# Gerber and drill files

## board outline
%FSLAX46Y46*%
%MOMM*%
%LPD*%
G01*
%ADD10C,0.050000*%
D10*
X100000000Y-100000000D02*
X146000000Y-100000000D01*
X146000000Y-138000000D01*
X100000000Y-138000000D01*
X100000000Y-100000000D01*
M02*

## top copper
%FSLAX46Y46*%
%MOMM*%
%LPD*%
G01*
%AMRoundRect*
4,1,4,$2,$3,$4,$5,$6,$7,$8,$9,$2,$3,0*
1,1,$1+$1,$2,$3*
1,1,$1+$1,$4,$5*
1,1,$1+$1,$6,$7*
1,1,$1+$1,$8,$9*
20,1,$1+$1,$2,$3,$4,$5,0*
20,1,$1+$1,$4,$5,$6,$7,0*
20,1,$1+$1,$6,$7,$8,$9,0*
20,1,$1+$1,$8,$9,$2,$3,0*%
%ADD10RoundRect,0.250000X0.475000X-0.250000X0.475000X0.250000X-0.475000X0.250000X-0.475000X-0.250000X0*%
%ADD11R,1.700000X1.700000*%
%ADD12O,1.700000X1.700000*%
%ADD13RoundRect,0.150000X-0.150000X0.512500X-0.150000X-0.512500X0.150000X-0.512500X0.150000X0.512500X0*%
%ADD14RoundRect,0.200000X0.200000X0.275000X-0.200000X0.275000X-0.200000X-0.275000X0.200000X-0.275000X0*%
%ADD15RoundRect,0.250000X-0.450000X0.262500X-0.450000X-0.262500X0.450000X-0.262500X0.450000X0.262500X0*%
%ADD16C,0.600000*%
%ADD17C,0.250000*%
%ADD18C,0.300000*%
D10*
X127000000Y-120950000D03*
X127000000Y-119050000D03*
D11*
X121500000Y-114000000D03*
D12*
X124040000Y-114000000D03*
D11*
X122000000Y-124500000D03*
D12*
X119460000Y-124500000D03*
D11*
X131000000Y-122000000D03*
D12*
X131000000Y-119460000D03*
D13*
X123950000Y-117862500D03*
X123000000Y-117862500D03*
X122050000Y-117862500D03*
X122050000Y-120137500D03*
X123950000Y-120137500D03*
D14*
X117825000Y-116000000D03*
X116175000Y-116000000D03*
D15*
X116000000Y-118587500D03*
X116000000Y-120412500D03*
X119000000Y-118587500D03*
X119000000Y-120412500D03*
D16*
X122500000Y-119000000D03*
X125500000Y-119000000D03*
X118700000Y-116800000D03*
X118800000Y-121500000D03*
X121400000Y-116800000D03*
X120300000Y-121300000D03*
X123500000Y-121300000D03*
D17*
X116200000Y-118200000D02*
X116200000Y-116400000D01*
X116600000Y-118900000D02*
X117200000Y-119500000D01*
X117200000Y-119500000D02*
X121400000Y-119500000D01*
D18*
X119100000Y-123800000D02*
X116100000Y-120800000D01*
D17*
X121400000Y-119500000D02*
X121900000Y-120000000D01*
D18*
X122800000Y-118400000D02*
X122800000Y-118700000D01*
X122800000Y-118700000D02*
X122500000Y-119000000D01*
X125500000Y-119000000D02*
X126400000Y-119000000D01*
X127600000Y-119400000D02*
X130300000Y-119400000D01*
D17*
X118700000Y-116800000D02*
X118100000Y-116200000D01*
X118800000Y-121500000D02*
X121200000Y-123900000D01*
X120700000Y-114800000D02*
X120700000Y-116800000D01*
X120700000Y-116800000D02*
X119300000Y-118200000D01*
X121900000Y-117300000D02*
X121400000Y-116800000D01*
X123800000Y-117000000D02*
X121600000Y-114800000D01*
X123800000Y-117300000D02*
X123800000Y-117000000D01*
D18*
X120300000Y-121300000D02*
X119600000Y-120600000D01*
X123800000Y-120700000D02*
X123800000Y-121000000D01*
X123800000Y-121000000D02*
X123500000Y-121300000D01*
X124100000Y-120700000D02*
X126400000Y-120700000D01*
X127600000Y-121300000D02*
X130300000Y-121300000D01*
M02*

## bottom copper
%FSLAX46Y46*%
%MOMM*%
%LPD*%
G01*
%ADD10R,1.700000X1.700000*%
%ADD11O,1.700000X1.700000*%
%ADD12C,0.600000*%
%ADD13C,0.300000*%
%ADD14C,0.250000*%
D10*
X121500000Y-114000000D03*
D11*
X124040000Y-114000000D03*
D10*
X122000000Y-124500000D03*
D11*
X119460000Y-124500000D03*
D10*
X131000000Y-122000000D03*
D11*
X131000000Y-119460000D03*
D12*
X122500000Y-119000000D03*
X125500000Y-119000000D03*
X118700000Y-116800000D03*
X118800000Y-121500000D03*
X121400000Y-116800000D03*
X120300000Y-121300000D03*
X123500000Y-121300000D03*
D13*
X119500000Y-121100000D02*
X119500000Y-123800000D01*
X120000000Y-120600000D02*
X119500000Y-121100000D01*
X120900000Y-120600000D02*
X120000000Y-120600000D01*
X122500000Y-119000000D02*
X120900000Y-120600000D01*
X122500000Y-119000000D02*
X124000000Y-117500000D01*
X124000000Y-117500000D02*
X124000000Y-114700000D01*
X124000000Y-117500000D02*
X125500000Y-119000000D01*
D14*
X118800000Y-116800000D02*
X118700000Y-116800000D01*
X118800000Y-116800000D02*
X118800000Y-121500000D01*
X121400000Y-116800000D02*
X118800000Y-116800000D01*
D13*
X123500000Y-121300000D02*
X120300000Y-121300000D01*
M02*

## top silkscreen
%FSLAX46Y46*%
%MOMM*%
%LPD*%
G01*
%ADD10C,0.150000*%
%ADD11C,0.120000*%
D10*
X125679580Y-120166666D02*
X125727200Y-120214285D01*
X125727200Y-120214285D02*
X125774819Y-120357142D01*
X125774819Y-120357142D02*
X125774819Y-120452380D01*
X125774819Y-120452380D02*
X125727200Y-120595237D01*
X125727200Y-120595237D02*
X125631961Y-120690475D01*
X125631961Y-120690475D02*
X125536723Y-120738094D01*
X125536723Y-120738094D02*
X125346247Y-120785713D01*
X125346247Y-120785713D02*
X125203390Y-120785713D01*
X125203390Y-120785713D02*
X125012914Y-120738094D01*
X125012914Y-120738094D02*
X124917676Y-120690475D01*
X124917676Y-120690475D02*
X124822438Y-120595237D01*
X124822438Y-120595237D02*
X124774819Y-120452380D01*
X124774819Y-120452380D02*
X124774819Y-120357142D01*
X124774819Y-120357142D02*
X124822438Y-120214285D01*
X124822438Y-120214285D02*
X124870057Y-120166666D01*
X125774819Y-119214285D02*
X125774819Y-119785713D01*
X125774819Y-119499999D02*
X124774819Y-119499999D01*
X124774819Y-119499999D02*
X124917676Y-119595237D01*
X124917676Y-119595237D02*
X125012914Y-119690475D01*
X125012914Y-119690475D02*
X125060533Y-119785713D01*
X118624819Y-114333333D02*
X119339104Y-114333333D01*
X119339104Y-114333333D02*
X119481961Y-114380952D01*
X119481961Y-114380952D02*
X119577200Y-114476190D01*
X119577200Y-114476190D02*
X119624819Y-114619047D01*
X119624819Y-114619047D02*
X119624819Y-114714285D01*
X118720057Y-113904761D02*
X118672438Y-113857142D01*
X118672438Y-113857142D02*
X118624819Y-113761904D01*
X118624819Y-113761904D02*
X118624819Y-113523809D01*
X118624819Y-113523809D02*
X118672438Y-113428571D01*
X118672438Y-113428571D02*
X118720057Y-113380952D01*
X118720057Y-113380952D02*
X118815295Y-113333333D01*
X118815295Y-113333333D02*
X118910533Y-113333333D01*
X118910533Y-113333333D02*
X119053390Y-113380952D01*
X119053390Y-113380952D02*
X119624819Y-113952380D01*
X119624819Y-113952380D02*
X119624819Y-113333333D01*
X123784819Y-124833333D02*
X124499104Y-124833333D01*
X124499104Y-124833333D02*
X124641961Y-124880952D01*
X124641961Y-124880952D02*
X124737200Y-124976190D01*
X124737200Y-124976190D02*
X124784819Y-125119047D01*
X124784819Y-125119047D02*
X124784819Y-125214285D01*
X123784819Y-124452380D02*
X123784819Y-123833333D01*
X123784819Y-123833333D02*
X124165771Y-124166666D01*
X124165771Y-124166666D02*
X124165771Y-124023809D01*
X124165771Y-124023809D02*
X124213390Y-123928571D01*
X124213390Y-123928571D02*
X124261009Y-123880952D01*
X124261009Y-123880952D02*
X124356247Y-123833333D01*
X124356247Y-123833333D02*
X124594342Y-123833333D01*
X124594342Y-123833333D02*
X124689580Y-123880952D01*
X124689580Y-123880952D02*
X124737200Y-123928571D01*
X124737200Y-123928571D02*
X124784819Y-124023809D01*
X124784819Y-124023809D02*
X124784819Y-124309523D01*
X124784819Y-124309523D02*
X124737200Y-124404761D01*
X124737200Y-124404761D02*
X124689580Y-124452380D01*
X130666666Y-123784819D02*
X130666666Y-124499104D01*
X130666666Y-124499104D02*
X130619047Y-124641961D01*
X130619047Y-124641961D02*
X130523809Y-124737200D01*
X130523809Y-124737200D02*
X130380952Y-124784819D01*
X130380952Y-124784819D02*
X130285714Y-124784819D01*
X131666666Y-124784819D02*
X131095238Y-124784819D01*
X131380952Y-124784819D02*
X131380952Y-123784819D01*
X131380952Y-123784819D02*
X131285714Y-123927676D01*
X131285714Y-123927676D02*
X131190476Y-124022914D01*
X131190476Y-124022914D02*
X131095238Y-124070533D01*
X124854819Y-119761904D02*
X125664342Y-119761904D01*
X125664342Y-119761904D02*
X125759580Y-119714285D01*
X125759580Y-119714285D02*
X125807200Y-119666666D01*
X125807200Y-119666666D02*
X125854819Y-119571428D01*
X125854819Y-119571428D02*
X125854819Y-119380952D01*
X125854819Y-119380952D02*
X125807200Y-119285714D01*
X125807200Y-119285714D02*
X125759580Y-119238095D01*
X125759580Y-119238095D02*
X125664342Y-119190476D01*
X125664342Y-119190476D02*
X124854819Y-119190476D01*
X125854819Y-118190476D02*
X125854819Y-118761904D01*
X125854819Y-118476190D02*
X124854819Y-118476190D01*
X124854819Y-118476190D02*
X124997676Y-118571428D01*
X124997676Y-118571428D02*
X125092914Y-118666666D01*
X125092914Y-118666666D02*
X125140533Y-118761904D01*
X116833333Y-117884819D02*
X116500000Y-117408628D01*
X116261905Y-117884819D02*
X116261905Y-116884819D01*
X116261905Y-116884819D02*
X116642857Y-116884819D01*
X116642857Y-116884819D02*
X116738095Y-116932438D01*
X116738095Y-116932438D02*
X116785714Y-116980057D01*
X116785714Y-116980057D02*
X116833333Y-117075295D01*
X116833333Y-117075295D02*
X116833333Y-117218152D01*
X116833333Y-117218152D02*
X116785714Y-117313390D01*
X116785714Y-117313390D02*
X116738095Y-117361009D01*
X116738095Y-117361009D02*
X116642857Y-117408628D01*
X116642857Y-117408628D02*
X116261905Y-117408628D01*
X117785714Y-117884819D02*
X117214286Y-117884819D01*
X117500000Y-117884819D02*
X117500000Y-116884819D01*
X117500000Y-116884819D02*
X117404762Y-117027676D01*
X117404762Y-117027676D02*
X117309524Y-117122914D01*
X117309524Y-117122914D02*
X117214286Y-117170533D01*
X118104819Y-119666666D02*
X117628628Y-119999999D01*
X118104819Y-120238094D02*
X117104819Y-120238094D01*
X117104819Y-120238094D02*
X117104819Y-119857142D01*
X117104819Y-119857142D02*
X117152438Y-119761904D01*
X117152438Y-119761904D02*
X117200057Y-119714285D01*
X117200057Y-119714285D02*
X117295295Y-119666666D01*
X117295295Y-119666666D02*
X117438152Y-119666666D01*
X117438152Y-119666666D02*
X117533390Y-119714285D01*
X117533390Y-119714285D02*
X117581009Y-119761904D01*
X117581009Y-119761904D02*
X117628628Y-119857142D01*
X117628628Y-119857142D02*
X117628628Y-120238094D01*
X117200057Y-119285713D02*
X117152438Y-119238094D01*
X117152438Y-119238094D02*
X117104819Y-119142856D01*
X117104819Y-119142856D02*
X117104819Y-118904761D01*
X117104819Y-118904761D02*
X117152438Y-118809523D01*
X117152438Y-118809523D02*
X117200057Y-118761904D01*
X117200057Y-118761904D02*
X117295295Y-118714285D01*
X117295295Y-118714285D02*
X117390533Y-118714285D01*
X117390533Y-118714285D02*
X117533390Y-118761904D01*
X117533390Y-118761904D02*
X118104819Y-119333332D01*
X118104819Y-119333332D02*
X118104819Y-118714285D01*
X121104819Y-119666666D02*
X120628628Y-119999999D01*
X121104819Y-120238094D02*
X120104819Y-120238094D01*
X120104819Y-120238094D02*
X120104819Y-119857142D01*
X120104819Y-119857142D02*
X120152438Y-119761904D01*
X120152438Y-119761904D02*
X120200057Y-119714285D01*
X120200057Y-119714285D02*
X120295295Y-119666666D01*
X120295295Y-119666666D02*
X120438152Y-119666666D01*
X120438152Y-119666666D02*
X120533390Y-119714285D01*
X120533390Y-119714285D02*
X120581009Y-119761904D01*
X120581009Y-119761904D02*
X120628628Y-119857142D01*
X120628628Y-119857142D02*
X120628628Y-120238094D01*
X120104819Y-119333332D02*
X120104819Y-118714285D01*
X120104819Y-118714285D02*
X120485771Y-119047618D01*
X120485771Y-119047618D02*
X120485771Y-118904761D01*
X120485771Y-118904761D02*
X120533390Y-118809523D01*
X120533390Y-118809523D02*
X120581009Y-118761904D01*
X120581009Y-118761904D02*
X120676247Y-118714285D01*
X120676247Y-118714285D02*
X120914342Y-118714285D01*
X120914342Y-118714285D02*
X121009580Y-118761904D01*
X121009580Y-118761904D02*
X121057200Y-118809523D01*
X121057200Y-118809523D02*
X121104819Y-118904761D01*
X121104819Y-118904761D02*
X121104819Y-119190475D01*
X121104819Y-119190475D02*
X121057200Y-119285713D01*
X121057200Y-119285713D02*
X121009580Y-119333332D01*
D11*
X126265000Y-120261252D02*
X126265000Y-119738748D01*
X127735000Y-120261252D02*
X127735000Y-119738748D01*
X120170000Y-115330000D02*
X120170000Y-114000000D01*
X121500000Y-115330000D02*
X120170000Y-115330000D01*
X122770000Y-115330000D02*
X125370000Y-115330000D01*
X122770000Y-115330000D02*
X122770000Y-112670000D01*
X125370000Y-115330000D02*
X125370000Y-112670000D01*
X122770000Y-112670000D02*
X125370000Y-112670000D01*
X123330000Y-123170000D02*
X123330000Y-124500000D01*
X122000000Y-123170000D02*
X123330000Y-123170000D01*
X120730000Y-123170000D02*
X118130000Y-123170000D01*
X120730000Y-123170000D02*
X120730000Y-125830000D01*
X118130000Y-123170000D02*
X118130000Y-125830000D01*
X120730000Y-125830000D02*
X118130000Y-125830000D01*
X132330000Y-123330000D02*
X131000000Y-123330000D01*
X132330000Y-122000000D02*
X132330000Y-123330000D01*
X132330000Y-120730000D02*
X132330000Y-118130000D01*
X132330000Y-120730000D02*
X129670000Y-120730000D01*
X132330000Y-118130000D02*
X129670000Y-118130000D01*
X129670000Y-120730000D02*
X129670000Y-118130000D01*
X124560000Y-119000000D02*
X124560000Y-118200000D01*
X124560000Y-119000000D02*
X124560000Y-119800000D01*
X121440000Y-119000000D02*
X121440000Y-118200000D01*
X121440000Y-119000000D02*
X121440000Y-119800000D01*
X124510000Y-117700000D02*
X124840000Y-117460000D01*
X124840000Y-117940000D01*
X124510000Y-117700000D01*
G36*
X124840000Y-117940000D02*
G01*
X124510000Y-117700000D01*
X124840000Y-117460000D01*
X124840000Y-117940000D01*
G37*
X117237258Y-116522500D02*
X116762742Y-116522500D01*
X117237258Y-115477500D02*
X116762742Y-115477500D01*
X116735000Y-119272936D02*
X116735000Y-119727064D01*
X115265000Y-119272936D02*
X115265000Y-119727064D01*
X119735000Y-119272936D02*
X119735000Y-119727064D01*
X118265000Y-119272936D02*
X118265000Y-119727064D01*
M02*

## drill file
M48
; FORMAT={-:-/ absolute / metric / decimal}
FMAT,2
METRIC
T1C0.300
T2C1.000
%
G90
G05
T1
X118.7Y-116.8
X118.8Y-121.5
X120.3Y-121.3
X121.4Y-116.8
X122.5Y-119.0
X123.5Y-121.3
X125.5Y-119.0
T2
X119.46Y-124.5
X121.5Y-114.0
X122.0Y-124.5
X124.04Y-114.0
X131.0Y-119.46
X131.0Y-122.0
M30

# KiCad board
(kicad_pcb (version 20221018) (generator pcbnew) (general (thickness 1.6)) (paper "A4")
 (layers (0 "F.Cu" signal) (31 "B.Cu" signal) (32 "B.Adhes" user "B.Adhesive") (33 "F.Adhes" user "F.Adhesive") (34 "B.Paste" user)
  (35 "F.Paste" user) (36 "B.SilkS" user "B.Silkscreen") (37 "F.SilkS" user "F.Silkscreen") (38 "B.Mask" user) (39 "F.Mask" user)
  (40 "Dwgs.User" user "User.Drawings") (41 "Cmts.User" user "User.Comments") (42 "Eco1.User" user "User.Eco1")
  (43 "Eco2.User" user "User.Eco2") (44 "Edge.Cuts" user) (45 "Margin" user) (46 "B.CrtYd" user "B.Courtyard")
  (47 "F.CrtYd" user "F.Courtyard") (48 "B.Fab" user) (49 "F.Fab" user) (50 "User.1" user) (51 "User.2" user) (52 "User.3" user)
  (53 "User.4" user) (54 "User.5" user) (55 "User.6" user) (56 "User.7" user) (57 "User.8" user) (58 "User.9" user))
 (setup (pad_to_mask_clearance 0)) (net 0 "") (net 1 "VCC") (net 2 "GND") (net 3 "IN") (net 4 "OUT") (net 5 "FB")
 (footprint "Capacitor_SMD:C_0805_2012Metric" (layer "F.Cu") (at 127 120 90)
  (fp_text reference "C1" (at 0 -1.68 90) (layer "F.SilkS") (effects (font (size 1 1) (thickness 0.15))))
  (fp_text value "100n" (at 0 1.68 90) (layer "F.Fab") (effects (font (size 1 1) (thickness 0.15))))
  (fp_line (start -0.261252 -0.735) (end 0.261252 -0.735) (stroke (width 0.12) (type solid)) (layer "F.SilkS"))
  (fp_line (start -0.261252 0.735) (end 0.261252 0.735) (stroke (width 0.12) (type solid)) (layer "F.SilkS"))
  (pad "1" smd roundrect (at -0.95 0 90) (size 1 1.45) (layers "F.Cu" "F.Paste" "F.Mask") (roundrect_rratio 0.25) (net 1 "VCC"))
  (pad "2" smd roundrect (at 0.95 0 90) (size 1 1.45) (layers "F.Cu" "F.Paste" "F.Mask") (roundrect_rratio 0.25) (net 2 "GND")))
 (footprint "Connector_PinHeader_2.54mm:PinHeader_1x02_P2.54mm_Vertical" (layer "F.Cu") (at 121.5 114 90)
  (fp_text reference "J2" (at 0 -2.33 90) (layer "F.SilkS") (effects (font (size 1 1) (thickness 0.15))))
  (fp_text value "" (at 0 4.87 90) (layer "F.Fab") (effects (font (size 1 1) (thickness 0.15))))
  (fp_line (start -1.33 -1.33) (end 0 -1.33) (stroke (width 0.12) (type solid)) (layer "F.SilkS"))
  (fp_line (start -1.33 0) (end -1.33 -1.33) (stroke (width 0.12) (type solid)) (layer "F.SilkS"))
  (fp_line (start -1.33 1.27) (end -1.33 3.87) (stroke (width 0.12) (type solid)) (layer "F.SilkS"))
  (fp_line (start -1.33 1.27) (end 1.33 1.27) (stroke (width 0.12) (type solid)) (layer "F.SilkS"))
  (fp_line (start -1.33 3.87) (end 1.33 3.87) (stroke (width 0.12) (type solid)) (layer "F.SilkS"))
  (fp_line (start 1.33 1.27) (end 1.33 3.87) (stroke (width 0.12) (type solid)) (layer "F.SilkS"))
  (pad "1" thru_hole rect (at 0 0 90) (size 1.7 1.7) (drill 1) (layers "*.Cu" "*.Mask") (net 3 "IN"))
  (pad "2" thru_hole oval (at 0 2.54 90) (size 1.7 1.7) (drill 1) (layers "*.Cu" "*.Mask") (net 2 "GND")))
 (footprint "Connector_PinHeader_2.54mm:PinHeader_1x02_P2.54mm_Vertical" (layer "F.Cu") (at 122 124.5 -90)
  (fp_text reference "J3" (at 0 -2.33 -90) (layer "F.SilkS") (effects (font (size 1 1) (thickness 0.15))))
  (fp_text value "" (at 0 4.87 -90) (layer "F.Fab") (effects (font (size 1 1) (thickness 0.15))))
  (fp_line (start -1.33 -1.33) (end 0 -1.33) (stroke (width 0.12) (type solid)) (layer "F.SilkS"))
  (fp_line (start -1.33 0) (end -1.33 -1.33) (stroke (width 0.12) (type solid)) (layer "F.SilkS"))
  (fp_line (start -1.33 1.27) (end -1.33 3.87) (stroke (width 0.12) (type solid)) (layer "F.SilkS"))
  (fp_line (start -1.33 1.27) (end 1.33 1.27) (stroke (width 0.12) (type solid)) (layer "F.SilkS"))
  (fp_line (start -1.33 3.87) (end 1.33 3.87) (stroke (width 0.12) (type solid)) (layer "F.SilkS"))
  (fp_line (start 1.33 1.27) (end 1.33 3.87) (stroke (width 0.12) (type solid)) (layer "F.SilkS"))
  (pad "1" thru_hole rect (at 0 0 270) (size 1.7 1.7) (drill 1) (layers "*.Cu" "*.Mask") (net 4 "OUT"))
  (pad "2" thru_hole oval (at 0 2.54 270) (size 1.7 1.7) (drill 1) (layers "*.Cu" "*.Mask") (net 2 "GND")))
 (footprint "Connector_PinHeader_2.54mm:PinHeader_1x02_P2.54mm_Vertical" (layer "F.Cu") (at 131 122 180)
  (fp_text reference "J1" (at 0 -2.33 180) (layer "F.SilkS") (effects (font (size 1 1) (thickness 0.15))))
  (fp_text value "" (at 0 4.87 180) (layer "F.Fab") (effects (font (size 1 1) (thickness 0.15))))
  (fp_line (start -1.33 -1.33) (end 0 -1.33) (stroke (width 0.12) (type solid)) (layer "F.SilkS"))
  (fp_line (start -1.33 0) (end -1.33 -1.33) (stroke (width 0.12) (type solid)) (layer "F.SilkS"))
  (fp_line (start -1.33 1.27) (end -1.33 3.87) (stroke (width 0.12) (type solid)) (layer "F.SilkS"))
  (fp_line (start -1.33 1.27) (end 1.33 1.27) (stroke (width 0.12) (type solid)) (layer "F.SilkS"))
  (fp_line (start -1.33 3.87) (end 1.33 3.87) (stroke (width 0.12) (type solid)) (layer "F.SilkS"))
  (fp_line (start 1.33 1.27) (end 1.33 3.87) (stroke (width 0.12) (type solid)) (layer "F.SilkS"))
  (pad "1" thru_hole rect (at 0 0 180) (size 1.7 1.7) (drill 1) (layers "*.Cu" "*.Mask") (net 1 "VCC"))
  (pad "2" thru_hole oval (at 0 2.54 180) (size 1.7 1.7) (drill 1) (layers "*.Cu" "*.Mask") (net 2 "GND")))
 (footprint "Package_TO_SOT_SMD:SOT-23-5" (layer "F.Cu") (at 123 119 -90)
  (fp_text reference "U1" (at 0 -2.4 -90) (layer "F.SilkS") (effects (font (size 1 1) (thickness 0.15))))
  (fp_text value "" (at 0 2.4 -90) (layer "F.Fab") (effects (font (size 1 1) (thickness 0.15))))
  (fp_line (start 0 -1.56) (end -0.8 -1.56) (stroke (width 0.12) (type solid)) (layer "F.SilkS"))
  (fp_line (start 0 -1.56) (end 0.8 -1.56) (stroke (width 0.12) (type solid)) (layer "F.SilkS"))
  (fp_line (start 0 1.56) (end -0.8 1.56) (stroke (width 0.12) (type solid)) (layer "F.SilkS"))
  (fp_line (start 0 1.56) (end 0.8 1.56) (stroke (width 0.12) (type solid)) (layer "F.SilkS"))
  (fp_poly
   (pts (xy -1.3 -1.51) (xy -1.54 -1.84) (xy -1.06 -1.84) (xy -1.3 -1.51)) (stroke (width 0.12) (type solid)) (fill solid) (layer "F.SilkS"))
  (pad "1" smd roundrect (at -1.1375 -0.95 270) (size 1.325 0.6) (layers "F.Cu" "F.Paste" "F.Mask") (roundrect_rratio 0.25) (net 3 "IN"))
  (pad "2" smd roundrect (at -1.1375 0 270) (size 1.325 0.6) (layers "F.Cu" "F.Paste" "F.Mask") (roundrect_rratio 0.25) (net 2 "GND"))
  (pad "3" smd roundrect (at -1.1375 0.95 270) (size 1.325 0.6) (layers "F.Cu" "F.Paste" "F.Mask") (roundrect_rratio 0.25) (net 4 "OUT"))
  (pad "4" smd roundrect (at 1.1375 0.95 270) (size 1.325 0.6) (layers "F.Cu" "F.Paste" "F.Mask") (roundrect_rratio 0.25) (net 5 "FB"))
  (pad "5" smd roundrect (at 1.1375 -0.95 270) (size 1.325 0.6) (layers "F.Cu" "F.Paste" "F.Mask") (roundrect_rratio 0.25) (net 1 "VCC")))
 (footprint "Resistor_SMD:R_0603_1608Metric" (layer "F.Cu") (at 117 116 180)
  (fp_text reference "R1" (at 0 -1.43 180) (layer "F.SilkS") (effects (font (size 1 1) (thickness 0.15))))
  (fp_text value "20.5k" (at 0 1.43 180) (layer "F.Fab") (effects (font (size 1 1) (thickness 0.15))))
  (fp_line (start -0.237258 -0.5225) (end 0.237258 -0.5225) (stroke (width 0.12) (type solid)) (layer "F.SilkS"))
  (fp_line (start -0.237258 0.5225) (end 0.237258 0.5225) (stroke (width 0.12) (type solid)) (layer "F.SilkS"))
  (pad "1" smd roundrect (at -0.825 0 180) (size 0.8 0.95) (layers "F.Cu" "F.Paste" "F.Mask") (roundrect_rratio 0.25) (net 4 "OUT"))
  (pad "2" smd roundrect (at 0.825 0 180) (size 0.8 0.95) (layers "F.Cu" "F.Paste" "F.Mask") (roundrect_rratio 0.25) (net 5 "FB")))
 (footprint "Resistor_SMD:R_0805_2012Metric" (layer "F.Cu") (at 116 119.5 -90)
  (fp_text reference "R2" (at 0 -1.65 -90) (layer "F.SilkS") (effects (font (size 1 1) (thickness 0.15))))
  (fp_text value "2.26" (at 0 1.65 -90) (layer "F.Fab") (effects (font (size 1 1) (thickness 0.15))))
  (fp_line (start -0.227064 -0.735) (end 0.227064 -0.735) (stroke (width 0.12) (type solid)) (layer "F.SilkS"))
  (fp_line (start -0.227064 0.735) (end 0.227064 0.735) (stroke (width 0.12) (type solid)) (layer "F.SilkS"))
  (pad "1" smd roundrect (at -0.9125 0 270) (size 1.025 1.4) (layers "F.Cu" "F.Paste" "F.Mask") (roundrect_rratio 0.243902) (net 5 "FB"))
  (pad "2" smd roundrect (at 0.9125 0 270) (size 1.025 1.4) (layers "F.Cu" "F.Paste" "F.Mask") (roundrect_rratio 0.243902) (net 2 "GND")))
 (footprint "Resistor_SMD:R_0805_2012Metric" (layer "F.Cu") (at 119 119.5 -90)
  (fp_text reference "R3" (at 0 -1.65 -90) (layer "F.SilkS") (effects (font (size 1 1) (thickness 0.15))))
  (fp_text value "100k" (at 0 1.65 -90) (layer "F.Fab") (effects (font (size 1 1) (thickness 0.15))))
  (fp_line (start -0.227064 -0.735) (end 0.227064 -0.735) (stroke (width 0.12) (type solid)) (layer "F.SilkS"))
  (fp_line (start -0.227064 0.735) (end 0.227064 0.735) (stroke (width 0.12) (type solid)) (layer "F.SilkS"))
  (pad "1" smd roundrect (at -0.9125 0 270) (size 1.025 1.4) (layers "F.Cu" "F.Paste" "F.Mask") (roundrect_rratio 0.243902) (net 3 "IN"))
  (pad "2" smd roundrect (at 0.9125 0 270) (size 1.025 1.4) (layers "F.Cu" "F.Paste" "F.Mask") (roundrect_rratio 0.243902) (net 1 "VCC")))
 (gr_rect (start 100 100) (end 146 138) (stroke (width 0.05) (type default)) (fill none) (layer "Edge.Cuts"))
 (segment (start 116.2 118.2) (end 116.2 116.4) (width 0.25) (layer "F.Cu") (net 5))
 (segment (start 116.6 118.9) (end 117.2 119.5) (width 0.25) (layer "F.Cu") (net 5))
 (segment (start 117.2 119.5) (end 121.4 119.5) (width 0.25) (layer "F.Cu") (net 5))
 (segment (start 119.1 123.8) (end 116.1 120.8) (width 0.3) (layer "F.Cu") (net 2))
 (segment (start 121.4 119.5) (end 121.9 120) (width 0.25) (layer "F.Cu") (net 5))
 (segment (start 122.8 118.4) (end 122.8 118.7) (width 0.3) (layer "F.Cu") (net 2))
 (segment (start 122.8 118.7) (end 122.5 119) (width 0.3) (layer "F.Cu") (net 2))
 (segment (start 125.5 119) (end 126.4 119) (width 0.3) (layer "F.Cu") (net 2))
 (segment (start 127.6 119.4) (end 130.3 119.4) (width 0.3) (layer "F.Cu") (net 2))
 (via (at 122.5 119) (size 0.6) (drill 0.3) (layers "F.Cu" "B.Cu") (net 2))
 (via (at 125.5 119) (size 0.6) (drill 0.3) (layers "F.Cu" "B.Cu") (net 2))
 (segment (start 118.7 116.8) (end 118.1 116.2) (width 0.25) (layer "F.Cu") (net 4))
 (segment (start 118.8 121.5) (end 121.2 123.9) (width 0.25) (layer "F.Cu") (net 4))
 (segment (start 119.5 121.1) (end 119.5 123.8) (width 0.3) (layer "B.Cu") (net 2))
 (segment (start 120 120.6) (end 119.5 121.1) (width 0.3) (layer "B.Cu") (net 2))
 (segment (start 120.7 114.8) (end 120.7 116.8) (width 0.25) (layer "F.Cu") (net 3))
 (segment (start 120.7 116.8) (end 119.3 118.2) (width 0.25) (layer "F.Cu") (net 3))
 (segment (start 120.9 120.6) (end 120 120.6) (width 0.3) (layer "B.Cu") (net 2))
 (segment (start 121.9 117.3) (end 121.4 116.8) (width 0.25) (layer "F.Cu") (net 4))
 (segment (start 122.5 119) (end 120.9 120.6) (width 0.3) (layer "B.Cu") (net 2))
 (segment (start 122.5 119) (end 124 117.5) (width 0.3) (layer "B.Cu") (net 2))
 (segment (start 123.8 117) (end 121.6 114.8) (width 0.25) (layer "F.Cu") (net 3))
 (segment (start 123.8 117.3) (end 123.8 117) (width 0.25) (layer "F.Cu") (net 3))
 (segment (start 124 117.5) (end 124 114.7) (width 0.3) (layer "B.Cu") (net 2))
 (segment (start 124 117.5) (end 125.5 119) (width 0.3) (layer "B.Cu") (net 2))
 (via (at 118.7 116.8) (size 0.6) (drill 0.3) (layers "F.Cu" "B.Cu") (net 4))
 (via (at 118.8 121.5) (size 0.6) (drill 0.3) (layers "F.Cu" "B.Cu") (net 4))
 (via (at 121.4 116.8) (size 0.6) (drill 0.3) (layers "F.Cu" "B.Cu") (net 4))
 (segment (start 118.8 116.8) (end 118.7 116.8) (width 0.25) (layer "B.Cu") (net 4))
 (segment (start 118.8 116.8) (end 118.8 121.5) (width 0.25) (layer "B.Cu") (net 4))
 (segment (start 120.3 121.3) (end 119.6 120.6) (width 0.3) (layer "F.Cu") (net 1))
 (segment (start 121.4 116.8) (end 118.8 116.8) (width 0.25) (layer "B.Cu") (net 4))
 (segment (start 123.8 120.7) (end 123.8 121) (width 0.3) (layer "F.Cu") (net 1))
 (segment (start 123.8 121) (end 123.5 121.3) (width 0.3) (layer "F.Cu") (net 1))
 (segment (start 124.1 120.7) (end 126.4 120.7) (width 0.3) (layer "F.Cu") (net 1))
 (segment (start 127.6 121.3) (end 130.3 121.3) (width 0.3) (layer "F.Cu") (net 1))
 (via (at 120.3 121.3) (size 0.6) (drill 0.3) (layers "F.Cu" "B.Cu") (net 1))
 (via (at 123.5 121.3) (size 0.6) (drill 0.3) (layers "F.Cu" "B.Cu") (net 1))
 (segment (start 123.5 121.3) (end 120.3 121.3) (width 0.3) (layer "B.Cu") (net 1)))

